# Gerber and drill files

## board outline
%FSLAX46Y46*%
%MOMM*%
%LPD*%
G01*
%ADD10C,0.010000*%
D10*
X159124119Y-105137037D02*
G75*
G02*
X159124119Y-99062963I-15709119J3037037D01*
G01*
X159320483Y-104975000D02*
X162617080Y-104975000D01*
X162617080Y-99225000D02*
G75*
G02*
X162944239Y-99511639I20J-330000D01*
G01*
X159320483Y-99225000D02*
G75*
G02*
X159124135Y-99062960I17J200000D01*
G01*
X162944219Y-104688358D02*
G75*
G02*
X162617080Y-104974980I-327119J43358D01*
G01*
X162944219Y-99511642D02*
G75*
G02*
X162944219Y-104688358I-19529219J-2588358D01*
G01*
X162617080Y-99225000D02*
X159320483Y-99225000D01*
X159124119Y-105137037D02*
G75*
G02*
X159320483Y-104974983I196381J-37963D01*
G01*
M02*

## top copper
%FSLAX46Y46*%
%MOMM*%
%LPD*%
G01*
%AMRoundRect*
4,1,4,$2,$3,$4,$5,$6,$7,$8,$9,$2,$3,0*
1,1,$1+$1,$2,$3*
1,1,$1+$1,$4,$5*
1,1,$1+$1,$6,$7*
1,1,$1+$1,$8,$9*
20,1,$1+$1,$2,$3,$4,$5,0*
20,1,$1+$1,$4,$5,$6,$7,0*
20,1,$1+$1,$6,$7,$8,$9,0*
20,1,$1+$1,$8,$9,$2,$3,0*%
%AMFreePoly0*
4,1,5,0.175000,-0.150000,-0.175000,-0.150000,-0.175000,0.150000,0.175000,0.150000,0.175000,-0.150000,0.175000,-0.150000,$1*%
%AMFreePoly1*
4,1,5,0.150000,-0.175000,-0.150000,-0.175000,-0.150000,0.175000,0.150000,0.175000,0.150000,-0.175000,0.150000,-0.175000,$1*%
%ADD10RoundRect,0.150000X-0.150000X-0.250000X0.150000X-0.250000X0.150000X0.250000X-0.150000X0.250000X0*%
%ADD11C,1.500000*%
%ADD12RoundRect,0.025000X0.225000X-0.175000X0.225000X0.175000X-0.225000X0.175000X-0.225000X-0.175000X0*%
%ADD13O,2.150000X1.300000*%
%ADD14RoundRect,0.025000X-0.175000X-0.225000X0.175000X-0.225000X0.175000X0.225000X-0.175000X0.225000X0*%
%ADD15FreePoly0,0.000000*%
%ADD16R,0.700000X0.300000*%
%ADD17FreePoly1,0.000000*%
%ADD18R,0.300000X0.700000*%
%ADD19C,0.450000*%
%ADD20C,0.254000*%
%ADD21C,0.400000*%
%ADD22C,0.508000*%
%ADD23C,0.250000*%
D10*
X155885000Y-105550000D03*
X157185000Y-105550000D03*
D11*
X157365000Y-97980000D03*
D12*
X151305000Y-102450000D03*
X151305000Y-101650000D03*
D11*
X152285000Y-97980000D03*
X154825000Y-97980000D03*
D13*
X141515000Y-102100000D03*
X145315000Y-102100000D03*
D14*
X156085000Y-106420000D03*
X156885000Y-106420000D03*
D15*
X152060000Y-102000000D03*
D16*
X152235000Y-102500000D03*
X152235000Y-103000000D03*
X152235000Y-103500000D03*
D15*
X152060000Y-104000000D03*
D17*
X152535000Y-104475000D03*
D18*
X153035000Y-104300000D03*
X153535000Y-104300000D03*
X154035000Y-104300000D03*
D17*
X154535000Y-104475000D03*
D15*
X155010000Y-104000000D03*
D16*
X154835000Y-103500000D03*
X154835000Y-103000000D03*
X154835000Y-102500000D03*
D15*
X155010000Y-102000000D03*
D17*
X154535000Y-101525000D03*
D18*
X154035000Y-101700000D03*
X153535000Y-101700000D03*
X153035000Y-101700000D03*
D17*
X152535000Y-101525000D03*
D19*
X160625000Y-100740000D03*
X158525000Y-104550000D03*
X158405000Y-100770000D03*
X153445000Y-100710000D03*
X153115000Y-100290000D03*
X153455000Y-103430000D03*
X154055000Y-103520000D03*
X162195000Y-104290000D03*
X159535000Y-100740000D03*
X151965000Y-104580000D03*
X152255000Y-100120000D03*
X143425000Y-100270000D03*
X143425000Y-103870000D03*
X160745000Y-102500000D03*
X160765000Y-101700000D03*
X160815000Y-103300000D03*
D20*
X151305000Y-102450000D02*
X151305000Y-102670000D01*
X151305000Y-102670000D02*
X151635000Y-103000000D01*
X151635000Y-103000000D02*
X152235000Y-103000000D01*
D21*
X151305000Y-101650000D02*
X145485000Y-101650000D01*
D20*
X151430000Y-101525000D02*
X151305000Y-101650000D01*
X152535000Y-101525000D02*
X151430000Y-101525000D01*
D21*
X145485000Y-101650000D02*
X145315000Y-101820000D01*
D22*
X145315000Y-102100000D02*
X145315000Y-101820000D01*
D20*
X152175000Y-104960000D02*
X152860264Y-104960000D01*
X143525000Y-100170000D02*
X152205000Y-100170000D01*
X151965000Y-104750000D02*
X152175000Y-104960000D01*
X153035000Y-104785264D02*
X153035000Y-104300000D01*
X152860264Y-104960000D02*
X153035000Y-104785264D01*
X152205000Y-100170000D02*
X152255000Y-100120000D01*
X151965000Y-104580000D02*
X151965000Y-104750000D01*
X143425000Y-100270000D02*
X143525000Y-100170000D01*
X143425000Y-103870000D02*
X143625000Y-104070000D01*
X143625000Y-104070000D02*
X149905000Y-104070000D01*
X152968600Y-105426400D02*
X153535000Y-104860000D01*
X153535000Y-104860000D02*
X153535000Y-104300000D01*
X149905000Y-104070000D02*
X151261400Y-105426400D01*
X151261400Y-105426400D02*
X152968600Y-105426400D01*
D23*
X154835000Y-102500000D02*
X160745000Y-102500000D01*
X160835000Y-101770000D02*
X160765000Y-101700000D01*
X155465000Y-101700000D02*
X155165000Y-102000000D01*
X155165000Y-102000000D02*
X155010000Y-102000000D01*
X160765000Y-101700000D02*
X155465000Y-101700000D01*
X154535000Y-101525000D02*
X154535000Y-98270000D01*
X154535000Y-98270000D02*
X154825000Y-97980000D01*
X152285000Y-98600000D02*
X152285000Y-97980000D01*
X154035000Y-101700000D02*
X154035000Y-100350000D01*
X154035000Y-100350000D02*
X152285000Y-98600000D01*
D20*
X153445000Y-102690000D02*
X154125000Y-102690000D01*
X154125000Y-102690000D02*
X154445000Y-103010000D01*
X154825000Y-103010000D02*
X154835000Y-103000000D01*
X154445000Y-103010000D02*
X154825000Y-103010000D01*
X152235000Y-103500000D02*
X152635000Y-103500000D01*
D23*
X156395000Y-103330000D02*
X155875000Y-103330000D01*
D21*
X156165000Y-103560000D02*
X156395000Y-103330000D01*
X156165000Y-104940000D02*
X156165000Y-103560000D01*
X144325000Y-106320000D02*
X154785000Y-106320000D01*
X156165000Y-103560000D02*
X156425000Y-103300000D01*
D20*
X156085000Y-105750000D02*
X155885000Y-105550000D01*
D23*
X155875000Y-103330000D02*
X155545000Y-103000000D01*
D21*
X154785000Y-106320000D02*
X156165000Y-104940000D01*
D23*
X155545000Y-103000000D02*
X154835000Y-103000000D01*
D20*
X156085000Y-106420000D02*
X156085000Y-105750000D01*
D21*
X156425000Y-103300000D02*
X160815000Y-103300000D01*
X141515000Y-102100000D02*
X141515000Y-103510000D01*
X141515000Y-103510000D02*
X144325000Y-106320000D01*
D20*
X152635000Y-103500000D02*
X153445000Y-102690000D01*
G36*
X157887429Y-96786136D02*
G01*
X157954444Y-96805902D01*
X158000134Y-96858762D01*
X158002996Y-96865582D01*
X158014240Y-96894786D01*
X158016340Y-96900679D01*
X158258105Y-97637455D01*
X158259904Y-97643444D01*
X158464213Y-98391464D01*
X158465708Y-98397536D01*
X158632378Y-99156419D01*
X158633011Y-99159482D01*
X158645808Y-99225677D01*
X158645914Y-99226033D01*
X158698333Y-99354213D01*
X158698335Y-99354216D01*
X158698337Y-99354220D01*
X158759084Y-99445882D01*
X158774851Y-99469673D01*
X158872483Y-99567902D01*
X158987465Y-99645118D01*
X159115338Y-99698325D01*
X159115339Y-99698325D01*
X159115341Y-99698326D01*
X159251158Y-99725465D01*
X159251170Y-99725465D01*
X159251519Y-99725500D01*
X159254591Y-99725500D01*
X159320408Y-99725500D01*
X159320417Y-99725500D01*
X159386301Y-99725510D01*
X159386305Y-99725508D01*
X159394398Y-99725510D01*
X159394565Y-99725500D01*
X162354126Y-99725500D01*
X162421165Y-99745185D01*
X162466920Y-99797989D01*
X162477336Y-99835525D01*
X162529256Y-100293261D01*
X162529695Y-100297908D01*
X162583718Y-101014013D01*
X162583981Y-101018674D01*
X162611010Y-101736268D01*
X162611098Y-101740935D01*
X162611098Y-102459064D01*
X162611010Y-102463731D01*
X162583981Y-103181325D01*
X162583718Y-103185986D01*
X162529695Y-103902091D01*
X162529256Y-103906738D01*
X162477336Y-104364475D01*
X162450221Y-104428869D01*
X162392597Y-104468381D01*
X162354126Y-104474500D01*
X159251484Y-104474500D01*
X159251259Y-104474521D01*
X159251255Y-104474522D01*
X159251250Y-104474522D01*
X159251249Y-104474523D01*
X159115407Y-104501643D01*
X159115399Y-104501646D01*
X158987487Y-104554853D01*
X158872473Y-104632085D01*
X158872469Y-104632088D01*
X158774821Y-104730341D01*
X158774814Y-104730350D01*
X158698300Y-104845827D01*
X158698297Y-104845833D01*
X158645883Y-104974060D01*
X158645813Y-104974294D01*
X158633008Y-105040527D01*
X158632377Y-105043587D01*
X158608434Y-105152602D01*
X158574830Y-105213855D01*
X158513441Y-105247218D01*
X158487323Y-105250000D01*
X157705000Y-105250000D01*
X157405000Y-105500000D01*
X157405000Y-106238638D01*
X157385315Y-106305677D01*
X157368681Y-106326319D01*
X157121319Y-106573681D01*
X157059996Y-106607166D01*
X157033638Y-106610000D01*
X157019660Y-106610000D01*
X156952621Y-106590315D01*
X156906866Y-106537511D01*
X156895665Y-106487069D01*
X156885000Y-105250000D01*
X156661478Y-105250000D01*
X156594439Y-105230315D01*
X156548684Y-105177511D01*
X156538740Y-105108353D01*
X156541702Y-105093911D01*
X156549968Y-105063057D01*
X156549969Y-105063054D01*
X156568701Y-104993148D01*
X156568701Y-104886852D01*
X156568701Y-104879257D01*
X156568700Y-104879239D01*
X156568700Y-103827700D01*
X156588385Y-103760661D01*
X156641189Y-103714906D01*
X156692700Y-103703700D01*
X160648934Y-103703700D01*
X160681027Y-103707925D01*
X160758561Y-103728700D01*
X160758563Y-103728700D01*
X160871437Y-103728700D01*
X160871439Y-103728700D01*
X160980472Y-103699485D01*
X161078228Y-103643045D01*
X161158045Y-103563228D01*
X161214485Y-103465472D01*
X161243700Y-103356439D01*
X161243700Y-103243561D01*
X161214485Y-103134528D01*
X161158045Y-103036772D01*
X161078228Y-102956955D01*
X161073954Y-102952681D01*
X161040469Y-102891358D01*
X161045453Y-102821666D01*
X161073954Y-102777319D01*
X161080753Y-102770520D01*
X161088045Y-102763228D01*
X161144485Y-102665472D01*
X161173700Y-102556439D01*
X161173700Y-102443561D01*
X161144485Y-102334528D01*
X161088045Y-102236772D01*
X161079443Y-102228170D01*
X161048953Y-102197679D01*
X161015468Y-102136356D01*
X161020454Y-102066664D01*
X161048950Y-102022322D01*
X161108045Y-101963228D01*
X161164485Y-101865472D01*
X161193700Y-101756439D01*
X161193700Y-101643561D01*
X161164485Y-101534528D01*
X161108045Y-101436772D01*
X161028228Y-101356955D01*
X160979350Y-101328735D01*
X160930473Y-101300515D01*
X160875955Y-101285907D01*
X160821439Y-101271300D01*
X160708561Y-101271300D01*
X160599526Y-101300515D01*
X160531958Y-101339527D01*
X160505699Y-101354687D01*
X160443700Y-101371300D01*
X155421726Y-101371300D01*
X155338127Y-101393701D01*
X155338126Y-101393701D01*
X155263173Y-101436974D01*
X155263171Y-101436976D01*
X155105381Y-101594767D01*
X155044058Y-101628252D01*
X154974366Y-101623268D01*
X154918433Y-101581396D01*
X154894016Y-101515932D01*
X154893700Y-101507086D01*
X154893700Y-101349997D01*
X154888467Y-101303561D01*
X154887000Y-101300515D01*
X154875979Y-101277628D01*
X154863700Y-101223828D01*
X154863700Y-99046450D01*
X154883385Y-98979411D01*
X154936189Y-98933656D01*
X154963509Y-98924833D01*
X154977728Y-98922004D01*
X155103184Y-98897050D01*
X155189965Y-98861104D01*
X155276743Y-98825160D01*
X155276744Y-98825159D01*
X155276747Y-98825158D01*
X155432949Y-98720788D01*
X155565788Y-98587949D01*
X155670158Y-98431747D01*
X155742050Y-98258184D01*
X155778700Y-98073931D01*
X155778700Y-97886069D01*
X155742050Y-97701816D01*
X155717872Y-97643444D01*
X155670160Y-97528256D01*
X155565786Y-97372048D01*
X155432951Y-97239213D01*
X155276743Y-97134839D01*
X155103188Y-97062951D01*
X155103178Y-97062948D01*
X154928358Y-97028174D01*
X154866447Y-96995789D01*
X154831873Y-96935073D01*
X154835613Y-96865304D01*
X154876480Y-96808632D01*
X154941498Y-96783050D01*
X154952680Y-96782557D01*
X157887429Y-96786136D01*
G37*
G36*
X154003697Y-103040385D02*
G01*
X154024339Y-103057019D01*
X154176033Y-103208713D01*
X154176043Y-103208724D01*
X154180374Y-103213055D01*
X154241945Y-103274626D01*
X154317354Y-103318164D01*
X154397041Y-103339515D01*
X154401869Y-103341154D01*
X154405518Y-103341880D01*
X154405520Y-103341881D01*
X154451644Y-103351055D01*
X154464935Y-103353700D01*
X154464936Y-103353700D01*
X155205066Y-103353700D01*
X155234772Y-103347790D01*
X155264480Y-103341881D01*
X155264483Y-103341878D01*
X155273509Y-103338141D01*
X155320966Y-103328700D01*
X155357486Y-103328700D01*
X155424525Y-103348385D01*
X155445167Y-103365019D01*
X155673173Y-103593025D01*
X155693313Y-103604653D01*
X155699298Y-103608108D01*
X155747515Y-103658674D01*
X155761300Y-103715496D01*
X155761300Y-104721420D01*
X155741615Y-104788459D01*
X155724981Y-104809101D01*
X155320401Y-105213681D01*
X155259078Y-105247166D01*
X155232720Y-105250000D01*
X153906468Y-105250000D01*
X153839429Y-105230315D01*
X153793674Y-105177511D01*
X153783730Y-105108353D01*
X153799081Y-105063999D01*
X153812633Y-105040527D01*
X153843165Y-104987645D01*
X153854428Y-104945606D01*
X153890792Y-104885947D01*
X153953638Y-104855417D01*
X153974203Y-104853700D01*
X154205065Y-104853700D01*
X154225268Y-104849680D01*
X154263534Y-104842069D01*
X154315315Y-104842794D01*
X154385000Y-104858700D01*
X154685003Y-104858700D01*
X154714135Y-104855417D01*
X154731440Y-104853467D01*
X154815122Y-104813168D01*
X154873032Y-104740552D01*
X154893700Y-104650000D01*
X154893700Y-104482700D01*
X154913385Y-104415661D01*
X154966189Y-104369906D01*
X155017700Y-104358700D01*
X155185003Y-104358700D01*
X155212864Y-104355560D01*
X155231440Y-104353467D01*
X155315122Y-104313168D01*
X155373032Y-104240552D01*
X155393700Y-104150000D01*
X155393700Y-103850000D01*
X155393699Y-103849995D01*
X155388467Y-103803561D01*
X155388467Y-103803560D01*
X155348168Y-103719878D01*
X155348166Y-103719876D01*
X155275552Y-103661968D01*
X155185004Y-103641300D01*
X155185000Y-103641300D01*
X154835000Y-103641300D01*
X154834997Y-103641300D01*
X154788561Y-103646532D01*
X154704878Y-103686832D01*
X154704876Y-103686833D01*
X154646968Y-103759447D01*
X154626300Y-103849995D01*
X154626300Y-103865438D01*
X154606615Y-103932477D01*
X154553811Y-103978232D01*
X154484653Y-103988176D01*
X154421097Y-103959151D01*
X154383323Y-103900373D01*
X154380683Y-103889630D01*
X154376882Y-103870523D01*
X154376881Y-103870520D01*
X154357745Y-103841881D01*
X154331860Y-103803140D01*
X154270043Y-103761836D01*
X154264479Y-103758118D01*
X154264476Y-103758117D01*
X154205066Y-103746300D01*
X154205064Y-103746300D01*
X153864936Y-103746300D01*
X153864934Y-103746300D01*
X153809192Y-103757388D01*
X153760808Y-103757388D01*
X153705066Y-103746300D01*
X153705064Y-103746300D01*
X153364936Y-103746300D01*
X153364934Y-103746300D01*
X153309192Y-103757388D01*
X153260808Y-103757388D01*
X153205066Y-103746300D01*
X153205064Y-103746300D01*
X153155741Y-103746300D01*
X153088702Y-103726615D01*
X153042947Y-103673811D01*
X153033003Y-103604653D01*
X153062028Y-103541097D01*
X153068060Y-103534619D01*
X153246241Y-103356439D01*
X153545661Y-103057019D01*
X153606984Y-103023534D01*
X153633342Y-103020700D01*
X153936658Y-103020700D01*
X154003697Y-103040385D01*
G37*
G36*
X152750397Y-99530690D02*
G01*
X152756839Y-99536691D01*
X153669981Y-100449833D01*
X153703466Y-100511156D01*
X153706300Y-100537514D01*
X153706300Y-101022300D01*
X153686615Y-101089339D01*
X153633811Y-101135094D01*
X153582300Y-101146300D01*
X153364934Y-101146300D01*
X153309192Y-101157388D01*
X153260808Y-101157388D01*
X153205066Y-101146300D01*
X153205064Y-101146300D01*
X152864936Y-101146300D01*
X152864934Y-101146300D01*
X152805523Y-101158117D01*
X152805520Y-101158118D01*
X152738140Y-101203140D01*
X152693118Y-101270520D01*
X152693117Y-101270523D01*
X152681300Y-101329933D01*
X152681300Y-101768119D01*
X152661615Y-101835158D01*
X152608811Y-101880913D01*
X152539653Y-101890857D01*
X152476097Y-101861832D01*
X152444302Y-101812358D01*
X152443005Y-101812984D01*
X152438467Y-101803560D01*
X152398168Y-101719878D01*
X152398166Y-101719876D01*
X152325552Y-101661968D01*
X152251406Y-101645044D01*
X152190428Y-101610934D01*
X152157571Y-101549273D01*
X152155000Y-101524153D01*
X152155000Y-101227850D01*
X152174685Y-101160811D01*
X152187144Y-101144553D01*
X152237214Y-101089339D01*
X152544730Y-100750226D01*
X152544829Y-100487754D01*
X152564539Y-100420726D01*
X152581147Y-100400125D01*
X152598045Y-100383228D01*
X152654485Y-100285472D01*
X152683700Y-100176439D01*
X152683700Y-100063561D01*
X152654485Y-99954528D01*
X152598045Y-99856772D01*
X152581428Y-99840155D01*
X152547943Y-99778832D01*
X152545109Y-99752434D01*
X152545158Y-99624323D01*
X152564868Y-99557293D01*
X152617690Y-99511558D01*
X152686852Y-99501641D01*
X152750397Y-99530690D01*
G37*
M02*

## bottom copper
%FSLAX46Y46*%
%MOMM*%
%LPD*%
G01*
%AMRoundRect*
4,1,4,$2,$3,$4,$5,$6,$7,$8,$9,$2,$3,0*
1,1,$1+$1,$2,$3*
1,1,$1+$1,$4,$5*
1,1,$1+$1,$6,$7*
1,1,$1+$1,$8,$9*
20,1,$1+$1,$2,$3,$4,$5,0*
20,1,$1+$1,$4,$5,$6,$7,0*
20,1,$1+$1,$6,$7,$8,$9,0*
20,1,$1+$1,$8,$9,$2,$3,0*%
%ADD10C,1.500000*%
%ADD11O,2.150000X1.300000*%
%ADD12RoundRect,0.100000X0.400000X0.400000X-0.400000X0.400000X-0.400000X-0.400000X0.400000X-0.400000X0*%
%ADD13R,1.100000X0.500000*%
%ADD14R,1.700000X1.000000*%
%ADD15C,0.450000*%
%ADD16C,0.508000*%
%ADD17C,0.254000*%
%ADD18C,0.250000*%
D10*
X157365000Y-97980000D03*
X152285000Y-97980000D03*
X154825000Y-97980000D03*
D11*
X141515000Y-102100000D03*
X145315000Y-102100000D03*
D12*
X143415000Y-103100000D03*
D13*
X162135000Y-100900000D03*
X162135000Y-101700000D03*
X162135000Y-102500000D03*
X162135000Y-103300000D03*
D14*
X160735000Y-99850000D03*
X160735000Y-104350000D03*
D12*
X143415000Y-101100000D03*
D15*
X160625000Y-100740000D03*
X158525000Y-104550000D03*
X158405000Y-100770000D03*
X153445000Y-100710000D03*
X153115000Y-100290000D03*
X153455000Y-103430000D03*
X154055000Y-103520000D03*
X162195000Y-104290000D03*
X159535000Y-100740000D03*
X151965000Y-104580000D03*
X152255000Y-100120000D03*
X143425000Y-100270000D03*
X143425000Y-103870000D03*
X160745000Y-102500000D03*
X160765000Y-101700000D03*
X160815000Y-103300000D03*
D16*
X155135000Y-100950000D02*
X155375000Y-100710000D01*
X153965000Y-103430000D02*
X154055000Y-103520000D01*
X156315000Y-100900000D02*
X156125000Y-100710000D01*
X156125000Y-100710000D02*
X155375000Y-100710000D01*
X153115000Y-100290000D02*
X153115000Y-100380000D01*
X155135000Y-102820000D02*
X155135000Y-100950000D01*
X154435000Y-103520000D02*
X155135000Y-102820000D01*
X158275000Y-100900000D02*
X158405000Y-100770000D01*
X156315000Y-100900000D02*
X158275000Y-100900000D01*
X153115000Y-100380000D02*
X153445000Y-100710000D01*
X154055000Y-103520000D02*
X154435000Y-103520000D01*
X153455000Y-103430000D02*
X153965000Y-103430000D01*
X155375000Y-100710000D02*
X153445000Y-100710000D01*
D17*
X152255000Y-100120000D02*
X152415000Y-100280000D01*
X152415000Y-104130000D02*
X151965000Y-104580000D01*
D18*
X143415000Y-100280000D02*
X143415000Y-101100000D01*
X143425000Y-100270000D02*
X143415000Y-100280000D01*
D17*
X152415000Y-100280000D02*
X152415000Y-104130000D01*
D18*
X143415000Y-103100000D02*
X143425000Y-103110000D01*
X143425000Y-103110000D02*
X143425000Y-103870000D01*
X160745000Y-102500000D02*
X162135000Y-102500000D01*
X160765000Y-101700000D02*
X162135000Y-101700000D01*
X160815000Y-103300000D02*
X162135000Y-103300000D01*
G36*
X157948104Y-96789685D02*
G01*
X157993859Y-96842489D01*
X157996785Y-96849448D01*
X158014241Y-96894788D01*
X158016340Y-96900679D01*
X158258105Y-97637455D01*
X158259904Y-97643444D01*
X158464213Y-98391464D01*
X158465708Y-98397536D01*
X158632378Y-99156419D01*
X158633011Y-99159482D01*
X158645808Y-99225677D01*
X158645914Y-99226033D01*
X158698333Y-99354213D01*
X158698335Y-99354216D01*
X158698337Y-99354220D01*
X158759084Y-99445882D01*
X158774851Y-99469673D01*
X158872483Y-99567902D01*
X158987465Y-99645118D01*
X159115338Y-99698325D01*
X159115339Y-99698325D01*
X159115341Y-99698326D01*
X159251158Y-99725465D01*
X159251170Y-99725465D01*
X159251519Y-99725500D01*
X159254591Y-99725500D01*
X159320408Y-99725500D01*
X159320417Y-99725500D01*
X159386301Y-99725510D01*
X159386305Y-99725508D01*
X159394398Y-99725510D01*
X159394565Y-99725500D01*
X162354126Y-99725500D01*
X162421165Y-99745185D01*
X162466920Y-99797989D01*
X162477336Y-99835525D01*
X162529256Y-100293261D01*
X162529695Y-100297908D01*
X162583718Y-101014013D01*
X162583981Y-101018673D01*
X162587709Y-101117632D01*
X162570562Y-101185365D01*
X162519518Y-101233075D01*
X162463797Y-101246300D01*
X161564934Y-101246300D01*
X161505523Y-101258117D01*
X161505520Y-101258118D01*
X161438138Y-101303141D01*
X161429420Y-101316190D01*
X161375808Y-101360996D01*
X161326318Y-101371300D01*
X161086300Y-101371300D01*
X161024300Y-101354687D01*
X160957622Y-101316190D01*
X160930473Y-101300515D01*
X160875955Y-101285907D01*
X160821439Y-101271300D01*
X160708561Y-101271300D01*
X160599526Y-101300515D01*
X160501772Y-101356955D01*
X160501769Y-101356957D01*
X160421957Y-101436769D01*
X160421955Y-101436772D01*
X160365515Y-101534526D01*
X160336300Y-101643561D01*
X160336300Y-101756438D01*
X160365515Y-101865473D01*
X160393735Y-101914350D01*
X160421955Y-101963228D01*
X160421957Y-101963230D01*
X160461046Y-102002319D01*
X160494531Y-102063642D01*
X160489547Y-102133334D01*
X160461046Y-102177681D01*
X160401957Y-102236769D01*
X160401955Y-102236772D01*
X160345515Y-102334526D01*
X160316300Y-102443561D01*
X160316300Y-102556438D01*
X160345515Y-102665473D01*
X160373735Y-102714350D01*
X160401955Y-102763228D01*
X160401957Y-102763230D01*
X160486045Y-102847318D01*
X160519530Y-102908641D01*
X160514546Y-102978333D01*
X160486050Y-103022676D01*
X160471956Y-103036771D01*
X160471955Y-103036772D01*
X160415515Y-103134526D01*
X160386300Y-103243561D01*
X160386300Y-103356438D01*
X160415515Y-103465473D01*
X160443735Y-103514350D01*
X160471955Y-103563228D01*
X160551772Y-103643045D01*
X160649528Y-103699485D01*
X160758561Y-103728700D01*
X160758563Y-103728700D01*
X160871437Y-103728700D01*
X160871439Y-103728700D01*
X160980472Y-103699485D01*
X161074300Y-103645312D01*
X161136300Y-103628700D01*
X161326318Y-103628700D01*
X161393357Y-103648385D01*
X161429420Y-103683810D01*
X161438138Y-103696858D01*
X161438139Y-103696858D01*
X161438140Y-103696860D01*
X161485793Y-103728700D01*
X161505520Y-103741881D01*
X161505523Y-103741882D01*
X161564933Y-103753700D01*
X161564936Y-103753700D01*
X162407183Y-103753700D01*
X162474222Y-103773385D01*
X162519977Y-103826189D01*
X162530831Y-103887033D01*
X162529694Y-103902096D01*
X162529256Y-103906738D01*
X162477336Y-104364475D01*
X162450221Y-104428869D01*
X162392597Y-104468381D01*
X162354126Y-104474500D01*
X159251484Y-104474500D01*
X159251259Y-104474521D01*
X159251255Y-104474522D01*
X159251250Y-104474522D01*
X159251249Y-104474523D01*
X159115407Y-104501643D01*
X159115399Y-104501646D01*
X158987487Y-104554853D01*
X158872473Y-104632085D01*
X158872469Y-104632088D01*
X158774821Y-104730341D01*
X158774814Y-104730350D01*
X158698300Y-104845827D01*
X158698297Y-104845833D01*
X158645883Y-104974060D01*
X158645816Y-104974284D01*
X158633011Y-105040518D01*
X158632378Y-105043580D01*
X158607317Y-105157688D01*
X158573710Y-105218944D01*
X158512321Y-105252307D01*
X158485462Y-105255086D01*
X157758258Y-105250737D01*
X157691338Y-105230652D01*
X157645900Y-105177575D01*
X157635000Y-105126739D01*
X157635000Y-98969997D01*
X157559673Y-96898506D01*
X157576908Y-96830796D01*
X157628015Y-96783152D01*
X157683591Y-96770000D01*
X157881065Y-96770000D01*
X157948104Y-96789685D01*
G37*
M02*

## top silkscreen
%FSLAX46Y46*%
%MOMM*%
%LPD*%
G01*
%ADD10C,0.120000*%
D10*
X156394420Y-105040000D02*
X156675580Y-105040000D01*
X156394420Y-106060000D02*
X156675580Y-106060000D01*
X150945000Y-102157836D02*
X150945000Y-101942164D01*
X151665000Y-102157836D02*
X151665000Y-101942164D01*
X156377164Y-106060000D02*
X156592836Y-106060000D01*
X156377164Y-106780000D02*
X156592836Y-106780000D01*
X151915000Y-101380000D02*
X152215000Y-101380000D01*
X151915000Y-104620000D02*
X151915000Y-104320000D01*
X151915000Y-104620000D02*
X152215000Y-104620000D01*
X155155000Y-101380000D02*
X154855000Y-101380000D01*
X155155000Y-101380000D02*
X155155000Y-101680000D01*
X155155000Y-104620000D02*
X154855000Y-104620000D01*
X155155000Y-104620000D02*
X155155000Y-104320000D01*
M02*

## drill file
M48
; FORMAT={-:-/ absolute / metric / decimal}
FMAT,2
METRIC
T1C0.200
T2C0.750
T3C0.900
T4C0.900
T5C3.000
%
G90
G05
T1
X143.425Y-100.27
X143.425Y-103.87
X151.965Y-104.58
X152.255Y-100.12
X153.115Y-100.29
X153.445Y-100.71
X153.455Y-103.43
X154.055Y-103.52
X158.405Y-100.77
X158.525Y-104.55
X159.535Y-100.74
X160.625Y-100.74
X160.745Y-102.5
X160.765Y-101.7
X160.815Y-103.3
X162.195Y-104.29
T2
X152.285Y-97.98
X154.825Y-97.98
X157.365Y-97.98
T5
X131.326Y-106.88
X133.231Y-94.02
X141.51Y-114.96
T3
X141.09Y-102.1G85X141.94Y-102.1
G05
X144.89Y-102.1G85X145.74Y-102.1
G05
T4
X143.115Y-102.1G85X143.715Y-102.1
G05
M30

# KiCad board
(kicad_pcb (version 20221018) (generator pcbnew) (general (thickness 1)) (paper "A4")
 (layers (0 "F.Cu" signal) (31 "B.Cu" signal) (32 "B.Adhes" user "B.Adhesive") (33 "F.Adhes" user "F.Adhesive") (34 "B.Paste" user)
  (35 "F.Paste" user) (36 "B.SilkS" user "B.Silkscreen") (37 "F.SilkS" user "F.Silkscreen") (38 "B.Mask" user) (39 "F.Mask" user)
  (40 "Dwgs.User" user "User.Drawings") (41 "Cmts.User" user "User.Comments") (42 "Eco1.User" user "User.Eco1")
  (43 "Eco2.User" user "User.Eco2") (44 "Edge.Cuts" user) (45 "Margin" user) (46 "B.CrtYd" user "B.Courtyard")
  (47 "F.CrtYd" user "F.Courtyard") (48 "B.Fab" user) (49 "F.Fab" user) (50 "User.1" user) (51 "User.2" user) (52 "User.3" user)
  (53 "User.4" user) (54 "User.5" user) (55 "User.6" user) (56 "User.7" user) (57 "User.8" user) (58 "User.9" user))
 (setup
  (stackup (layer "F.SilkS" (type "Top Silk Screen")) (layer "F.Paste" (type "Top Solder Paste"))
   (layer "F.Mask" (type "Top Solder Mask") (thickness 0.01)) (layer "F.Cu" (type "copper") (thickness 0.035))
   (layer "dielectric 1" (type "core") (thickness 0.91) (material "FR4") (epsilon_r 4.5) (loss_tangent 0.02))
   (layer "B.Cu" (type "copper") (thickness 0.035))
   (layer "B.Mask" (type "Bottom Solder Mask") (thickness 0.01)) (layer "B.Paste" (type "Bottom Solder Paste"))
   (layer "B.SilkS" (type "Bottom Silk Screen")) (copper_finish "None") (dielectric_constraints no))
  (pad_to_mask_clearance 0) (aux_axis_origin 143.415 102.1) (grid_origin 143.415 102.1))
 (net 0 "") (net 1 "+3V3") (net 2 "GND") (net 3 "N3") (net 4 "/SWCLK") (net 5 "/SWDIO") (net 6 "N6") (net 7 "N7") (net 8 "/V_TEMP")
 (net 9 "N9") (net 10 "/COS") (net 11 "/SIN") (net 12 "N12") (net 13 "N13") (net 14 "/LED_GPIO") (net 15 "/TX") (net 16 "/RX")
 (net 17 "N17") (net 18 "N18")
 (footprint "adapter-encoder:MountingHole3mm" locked (layer "F.Cu") (at 141.509772 114.959631)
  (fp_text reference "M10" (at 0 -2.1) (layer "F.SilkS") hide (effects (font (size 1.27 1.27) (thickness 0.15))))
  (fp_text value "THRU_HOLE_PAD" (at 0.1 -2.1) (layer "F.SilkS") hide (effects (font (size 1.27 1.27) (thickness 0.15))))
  (pad "" np_thru_hole oval locked (at 0 0) (size 3 3) (drill 3) (layers "*.Mask") (thermal_bridge_angle 45)))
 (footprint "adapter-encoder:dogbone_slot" (layer "F.Cu") (at 143.415 102.1)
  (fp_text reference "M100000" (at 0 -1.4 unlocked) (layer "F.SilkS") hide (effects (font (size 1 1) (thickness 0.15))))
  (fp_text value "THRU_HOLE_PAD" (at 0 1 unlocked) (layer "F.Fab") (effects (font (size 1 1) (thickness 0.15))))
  (pad "" np_thru_hole oval (at 0 0) (size 1.5 0.9) (drill oval 1.5 0.9) (layers "*.Mask") (thermal_bridge_angle 45)))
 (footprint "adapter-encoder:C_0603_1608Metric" (layer "F.Cu") (at 156.535 105.55)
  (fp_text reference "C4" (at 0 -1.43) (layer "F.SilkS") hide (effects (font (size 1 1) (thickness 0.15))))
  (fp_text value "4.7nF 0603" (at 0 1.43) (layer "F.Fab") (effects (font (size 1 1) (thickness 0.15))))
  (fp_line (start -0.14058 -0.51) (end 0.14058 -0.51) (stroke (width 0.12) (type solid)) (layer "F.SilkS"))
  (fp_line (start -0.14058 0.51) (end 0.14058 0.51) (stroke (width 0.12) (type solid)) (layer "F.SilkS"))
  (pad "1" smd roundrect (at -0.65 0) (size 0.6 0.8) (layers "F.Cu" "F.Paste" "F.Mask") (roundrect_rratio 0.25) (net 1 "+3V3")
   (solder_mask_margin 0.0508))
  (pad "2" smd roundrect (at 0.65 0) (size 0.6 0.8) (layers "F.Cu" "F.Paste" "F.Mask") (roundrect_rratio 0.25) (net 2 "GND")
   (solder_mask_margin 0.0508)))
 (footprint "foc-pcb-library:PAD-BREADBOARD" (layer "F.Cu") (at 157.365 97.98)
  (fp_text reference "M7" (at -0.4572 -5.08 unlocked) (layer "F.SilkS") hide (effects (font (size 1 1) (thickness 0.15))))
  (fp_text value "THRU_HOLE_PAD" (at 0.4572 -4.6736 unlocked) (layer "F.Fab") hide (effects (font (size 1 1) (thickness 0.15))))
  (pad "1" thru_hole circle (at 0 0) (size 1.5 1.5) (drill 0.75) (layers "*.Cu" "*.Mask") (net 2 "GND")))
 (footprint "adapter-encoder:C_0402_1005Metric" (layer "F.Cu") (at 151.305 102.05 90)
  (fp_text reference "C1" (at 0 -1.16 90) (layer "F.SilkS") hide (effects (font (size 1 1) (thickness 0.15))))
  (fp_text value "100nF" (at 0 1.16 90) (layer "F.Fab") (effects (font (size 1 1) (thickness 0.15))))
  (fp_line (start -0.107836 -0.36) (end 0.107836 -0.36) (stroke (width 0.12) (type solid)) (layer "F.SilkS"))
  (fp_line (start -0.107836 0.36) (end 0.107836 0.36) (stroke (width 0.12) (type solid)) (layer "F.SilkS"))
  (pad "1" smd roundrect (at -0.4 0 90) (size 0.4 0.5) (layers "F.Cu" "F.Paste" "F.Mask") (roundrect_rratio 0.0625) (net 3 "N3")
   (solder_mask_margin 0.0508))
  (pad "2" smd roundrect (at 0.4 0 90) (size 0.4 0.5) (layers "F.Cu" "F.Paste" "F.Mask") (roundrect_rratio 0.0625) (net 2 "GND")
   (solder_mask_margin 0.0508)))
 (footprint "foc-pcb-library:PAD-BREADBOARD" (layer "F.Cu") (at 152.285 97.98)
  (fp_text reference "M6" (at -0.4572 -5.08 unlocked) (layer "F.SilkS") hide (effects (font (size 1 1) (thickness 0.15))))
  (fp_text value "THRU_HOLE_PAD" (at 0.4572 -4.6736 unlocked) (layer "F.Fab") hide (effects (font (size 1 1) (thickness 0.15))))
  (pad "1" thru_hole circle (at 0 0) (size 1.5 1.5) (drill 0.75) (layers "*.Cu" "*.Mask") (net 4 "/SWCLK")))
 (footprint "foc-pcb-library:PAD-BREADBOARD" (layer "F.Cu") (at 154.825 97.98)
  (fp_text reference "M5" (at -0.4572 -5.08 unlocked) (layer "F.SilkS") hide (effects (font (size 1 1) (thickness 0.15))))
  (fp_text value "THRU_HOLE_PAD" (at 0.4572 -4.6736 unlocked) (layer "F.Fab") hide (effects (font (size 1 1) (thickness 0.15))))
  (pad "1" thru_hole circle (at 0 0) (size 1.5 1.5) (drill 0.75) (layers "*.Cu" "*.Mask") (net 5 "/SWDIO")))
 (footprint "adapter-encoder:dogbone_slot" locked (layer "F.Cu") (at 141.515 102.1)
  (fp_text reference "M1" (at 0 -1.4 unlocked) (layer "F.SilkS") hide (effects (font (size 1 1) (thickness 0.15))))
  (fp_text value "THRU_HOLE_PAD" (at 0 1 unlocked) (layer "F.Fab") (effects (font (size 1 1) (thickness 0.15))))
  (pad "1" thru_hole oval locked (at 0 0) (size 2.15 1.3) (drill oval 1.75 0.9) (layers "*.Cu" "*.Mask") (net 1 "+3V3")
   (thermal_bridge_angle 45)))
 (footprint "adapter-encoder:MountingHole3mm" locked (layer "F.Cu") (at 133.230847 94.02021)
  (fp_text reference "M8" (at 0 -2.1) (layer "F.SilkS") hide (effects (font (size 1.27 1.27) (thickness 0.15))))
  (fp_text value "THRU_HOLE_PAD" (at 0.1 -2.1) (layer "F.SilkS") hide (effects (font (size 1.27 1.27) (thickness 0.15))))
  (pad "" np_thru_hole oval locked (at 0 0) (size 3 3) (drill 3) (layers "*.Mask") (thermal_bridge_angle 45)))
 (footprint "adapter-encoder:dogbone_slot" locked (layer "F.Cu") (at 145.315 102.1)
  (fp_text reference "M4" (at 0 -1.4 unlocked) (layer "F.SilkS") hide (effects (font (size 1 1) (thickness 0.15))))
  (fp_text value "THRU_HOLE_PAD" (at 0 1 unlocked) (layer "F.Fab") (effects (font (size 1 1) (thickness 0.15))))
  (pad "1" thru_hole oval locked (at 0 0) (size 2.15 1.3) (drill oval 1.75 0.9) (layers "*.Cu" "*.Mask") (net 2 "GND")
   (thermal_bridge_angle 45)))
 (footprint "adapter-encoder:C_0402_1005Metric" (layer "F.Cu") (at 156.485 106.42)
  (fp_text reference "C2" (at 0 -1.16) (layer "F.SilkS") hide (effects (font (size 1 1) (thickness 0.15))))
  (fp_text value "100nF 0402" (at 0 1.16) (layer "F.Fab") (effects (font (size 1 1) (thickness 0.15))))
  (fp_line (start -0.107836 -0.36) (end 0.107836 -0.36) (stroke (width 0.12) (type solid)) (layer "F.SilkS"))
  (fp_line (start -0.107836 0.36) (end 0.107836 0.36) (stroke (width 0.12) (type solid)) (layer "F.SilkS"))
  (pad "1" smd roundrect (at -0.4 0) (size 0.4 0.5) (layers "F.Cu" "F.Paste" "F.Mask") (roundrect_rratio 0.0625) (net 1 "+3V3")
   (solder_mask_margin 0.0508))
  (pad "2" smd roundrect (at 0.4 0) (size 0.4 0.5) (layers "F.Cu" "F.Paste" "F.Mask") (roundrect_rratio 0.0625) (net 2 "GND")
   (solder_mask_margin 0.0508)))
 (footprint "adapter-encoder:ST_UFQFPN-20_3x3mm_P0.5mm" (layer "F.Cu") (at 153.535 103)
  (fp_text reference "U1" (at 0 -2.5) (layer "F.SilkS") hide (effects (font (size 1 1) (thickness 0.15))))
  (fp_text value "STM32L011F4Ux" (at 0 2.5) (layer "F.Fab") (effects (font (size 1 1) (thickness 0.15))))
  (fp_line (start -1.62 -1.62) (end -1.32 -1.62) (stroke (width 0.12) (type solid)) (layer "F.SilkS"))
  (fp_line (start -1.62 1.62) (end -1.62 1.32) (stroke (width 0.12) (type solid)) (layer "F.SilkS"))
  (fp_line (start -1.62 1.62) (end -1.32 1.62) (stroke (width 0.12) (type solid)) (layer "F.SilkS"))
  (fp_line (start 1.62 -1.62) (end 1.32 -1.62) (stroke (width 0.12) (type solid)) (layer "F.SilkS"))
  (fp_line (start 1.62 -1.62) (end 1.62 -1.32) (stroke (width 0.12) (type solid)) (layer "F.SilkS"))
  (fp_line (start 1.62 1.62) (end 1.32 1.62) (stroke (width 0.12) (type solid)) (layer "F.SilkS"))
  (fp_line (start 1.62 1.62) (end 1.62 1.32) (stroke (width 0.12) (type solid)) (layer "F.SilkS"))
  (pad "1" smd custom (at -1.475 -1) (size 0.35 0.3) (layers "F.Cu" "F.Paste" "F.Mask") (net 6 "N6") (zone_connect 2)
   (options (clearance outline) (anchor rect)) (primitives))
  (pad "2" smd rect (at -1.3 -0.5) (size 0.7 0.3) (layers "F.Cu" "F.Paste" "F.Mask") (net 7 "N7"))
  (pad "3" smd rect (at -1.3 0) (size 0.7 0.3) (layers "F.Cu" "F.Paste" "F.Mask") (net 3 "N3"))
  (pad "4" smd rect (at -1.3 0.5) (size 0.7 0.3) (layers "F.Cu" "F.Paste" "F.Mask") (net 1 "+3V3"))
  (pad "5" smd custom (at -1.475 1) (size 0.35 0.3) (layers "F.Cu" "F.Paste" "F.Mask") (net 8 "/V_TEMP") (zone_connect 2)
   (options (clearance outline) (anchor rect)) (primitives))
  (pad "6" smd custom (at -1 1.475) (size 0.3 0.35) (layers "F.Cu" "F.Paste" "F.Mask") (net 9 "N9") (zone_connect 2)
   (options (clearance outline) (anchor rect)) (primitives))
  (pad "7" smd rect (at -0.5 1.3) (size 0.3 0.7) (layers "F.Cu" "F.Paste" "F.Mask") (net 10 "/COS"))
  (pad "8" smd rect (at 0 1.3) (size 0.3 0.7) (layers "F.Cu" "F.Paste" "F.Mask") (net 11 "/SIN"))
  (pad "9" smd rect (at 0.5 1.3) (size 0.3 0.7) (layers "F.Cu" "F.Paste" "F.Mask") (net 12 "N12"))
  (pad "10" smd custom (at 1 1.475) (size 0.3 0.35) (layers "F.Cu" "F.Paste" "F.Mask") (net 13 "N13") (zone_connect 2)
   (options (clearance outline) (anchor rect)) (primitives))
  (pad "11" smd custom (at 1.475 1) (size 0.35 0.3) (layers "F.Cu" "F.Paste" "F.Mask") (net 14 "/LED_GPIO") (zone_connect 2)
   (options (clearance outline) (anchor rect)) (primitives))
  (pad "12" smd rect (at 1.3 0.5) (size 0.7 0.3) (layers "F.Cu" "F.Paste" "F.Mask") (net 2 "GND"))
  (pad "13" smd rect (at 1.3 0) (size 0.7 0.3) (layers "F.Cu" "F.Paste" "F.Mask") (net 1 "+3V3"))
  (pad "14" smd rect (at 1.3 -0.5) (size 0.7 0.3) (layers "F.Cu" "F.Paste" "F.Mask") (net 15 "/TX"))
  (pad "15" smd custom (at 1.475 -1) (size 0.35 0.3) (layers "F.Cu" "F.Paste" "F.Mask") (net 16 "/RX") (zone_connect 2)
   (options (clearance outline) (anchor rect)) (primitives))
  (pad "16" smd custom (at 1 -1.475) (size 0.3 0.35) (layers "F.Cu" "F.Paste" "F.Mask") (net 5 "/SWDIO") (zone_connect 2)
   (options (clearance outline) (anchor rect)) (primitives))
  (pad "17" smd rect (at 0.5 -1.3) (size 0.3 0.7) (layers "F.Cu" "F.Paste" "F.Mask") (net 4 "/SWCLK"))
  (pad "18" smd rect (at 0 -1.3) (size 0.3 0.7) (layers "F.Cu" "F.Paste" "F.Mask") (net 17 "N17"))
  (pad "19" smd rect (at -0.5 -1.3) (size 0.3 0.7) (layers "F.Cu" "F.Paste" "F.Mask") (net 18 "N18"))
  (pad "20" smd custom (at -1 -1.475) (size 0.3 0.35) (layers "F.Cu" "F.Paste" "F.Mask") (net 2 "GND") (zone_connect 2)
   (options (clearance outline) (anchor rect)) (primitives)))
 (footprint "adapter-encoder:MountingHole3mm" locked (layer "F.Cu") (at 131.325619 106.87984)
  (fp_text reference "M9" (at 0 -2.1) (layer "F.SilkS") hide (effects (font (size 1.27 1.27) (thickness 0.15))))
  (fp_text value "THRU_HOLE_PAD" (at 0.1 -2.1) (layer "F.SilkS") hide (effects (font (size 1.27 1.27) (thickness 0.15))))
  (pad "" np_thru_hole oval locked (at 0 0) (size 3 3) (drill 3) (layers "*.Mask") (thermal_bridge_angle 45)))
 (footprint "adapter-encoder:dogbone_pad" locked (layer "B.Cu") (at 143.415 103.1 180)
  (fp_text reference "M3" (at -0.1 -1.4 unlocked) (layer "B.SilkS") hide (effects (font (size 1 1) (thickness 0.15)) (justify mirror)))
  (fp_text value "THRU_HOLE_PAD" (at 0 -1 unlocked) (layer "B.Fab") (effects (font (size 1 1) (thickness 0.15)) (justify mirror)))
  (pad "1" smd roundrect locked (at 0 0 180) (size 1 1) (layers "B.Cu" "B.Paste" "B.Mask") (roundrect_rratio 0.1) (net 11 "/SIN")
   (thermal_bridge_angle 45)))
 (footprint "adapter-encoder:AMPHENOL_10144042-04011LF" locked (layer "B.Cu") (at 162.135 102.1 90)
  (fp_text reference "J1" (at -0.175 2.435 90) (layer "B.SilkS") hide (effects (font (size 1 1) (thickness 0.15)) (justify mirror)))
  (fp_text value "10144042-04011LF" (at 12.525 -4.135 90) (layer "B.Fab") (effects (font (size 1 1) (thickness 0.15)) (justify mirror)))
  (pad "1" smd rect locked (at 1.2 0 90) (size 0.5 1.1) (layers "B.Cu" "B.Paste" "B.Mask") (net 2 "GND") (solder_mask_margin 0.102))
  (pad "2" smd rect locked (at 0.4 0 90) (size 0.5 1.1) (layers "B.Cu" "B.Paste" "B.Mask") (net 16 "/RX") (solder_mask_margin 0.102))
  (pad "3" smd rect locked (at -0.4 0 90) (size 0.5 1.1) (layers "B.Cu" "B.Paste" "B.Mask") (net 15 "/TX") (solder_mask_margin 0.102))
  (pad "4" smd rect locked (at -1.2 0 90) (size 0.5 1.1) (layers "B.Cu" "B.Paste" "B.Mask") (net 1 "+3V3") (solder_mask_margin 0.102))
  (pad "S1" smd rect locked (at 2.25 -1.4 90) (size 1 1.7) (layers "B.Cu" "B.Paste" "B.Mask") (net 2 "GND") (solder_mask_margin 0.102))
  (pad "S2" smd rect locked (at -2.25 -1.4 90) (size 1 1.7) (layers "B.Cu" "B.Paste" "B.Mask") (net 2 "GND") (solder_mask_margin 0.102)))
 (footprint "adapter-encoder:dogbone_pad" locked (layer "B.Cu") (at 143.415 101.1 180)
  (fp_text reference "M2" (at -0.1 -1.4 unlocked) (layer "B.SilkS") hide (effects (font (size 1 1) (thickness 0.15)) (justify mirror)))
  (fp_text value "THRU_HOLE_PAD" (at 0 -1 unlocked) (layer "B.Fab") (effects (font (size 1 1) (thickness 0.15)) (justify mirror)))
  (pad "1" smd roundrect locked (at 0 0 180) (size 1 1) (layers "B.Cu" "B.Paste" "B.Mask") (roundrect_rratio 0.1) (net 10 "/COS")
   (thermal_bridge_angle 45)))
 (gr_arc locked (start 159.124119 105.137037) (mid 127.415 102.1) (end 159.124119 99.062963) (stroke (width 0.01) (type solid))
  (layer "Edge.Cuts"))
 (gr_line locked (start 159.320483 104.975) (end 162.61708 104.975) (stroke (width 0.01) (type solid)) (layer "Edge.Cuts"))
 (gr_arc locked (start 162.61708 99.225) (mid 162.834568 99.306791) (end 162.944219 99.511642) (stroke (width 0.01) (type solid))
  (layer "Edge.Cuts"))
 (gr_arc locked (start 159.320483 99.225) (mid 159.193198 99.179254) (end 159.124119 99.062963) (stroke (width 0.01) (type solid))
  (layer "Edge.Cuts"))
 (gr_arc locked (start 162.944219 104.688358) (mid 162.834555 104.893194) (end 162.61708 104.975) (stroke (width 0.01) (type solid))
  (layer "Edge.Cuts"))
 (gr_arc locked (start 162.944219 99.511642) (mid 163.115 102.1) (end 162.944219 104.688358) (stroke (width 0.01) (type solid))
  (layer "Edge.Cuts"))
 (gr_line locked (start 162.61708 99.225) (end 159.320483 99.225) (stroke (width 0.01) (type solid)) (layer "Edge.Cuts"))
 (gr_arc locked (start 159.124119 105.137037) (mid 159.193188 105.020733) (end 159.320483 104.975) (stroke (width 0.01) (type solid))
  (layer "Edge.Cuts"))
 (segment (start 151.305 102.45) (end 151.305 102.67) (width 0.254) (layer "F.Cu") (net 3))
 (segment (start 151.305 102.67) (end 151.635 103) (width 0.254) (layer "F.Cu") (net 3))
 (segment (start 151.635 103) (end 152.235 103) (width 0.254) (layer "F.Cu") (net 3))
 (segment (start 151.305 101.65) (end 145.485 101.65) (width 0.4) (layer "F.Cu") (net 2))
 (segment (start 151.43 101.525) (end 151.305 101.65) (width 0.254) (layer "F.Cu") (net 2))
 (segment (start 152.535 101.525) (end 151.43 101.525) (width 0.254) (layer "F.Cu") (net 2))
 (segment (start 145.485 101.65) (end 145.315 101.82) (width 0.4) (layer "F.Cu") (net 2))
 (segment (start 145.315 102.1) (end 145.315 101.82) (width 0.508) (layer "F.Cu") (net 2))
 (via (at 160.625 100.74) (size 0.45) (drill 0.2) (layers "F.Cu" "B.Cu") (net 2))
 (via (at 158.525 104.55) (size 0.45) (drill 0.2) (layers "F.Cu" "B.Cu") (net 2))
 (via (at 158.405 100.77) (size 0.45) (drill 0.2) (layers "F.Cu" "B.Cu") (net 2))
 (via (at 153.445 100.71) (size 0.45) (drill 0.2) (layers "F.Cu" "B.Cu") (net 2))
 (via (at 153.115 100.29) (size 0.45) (drill 0.2) (layers "F.Cu" "B.Cu") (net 2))
 (via (at 153.455 103.43) (size 0.45) (drill 0.2) (layers "F.Cu" "B.Cu") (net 2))
 (via (at 154.055 103.52) (size 0.45) (drill 0.2) (layers "F.Cu" "B.Cu") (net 2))
 (via (at 162.195 104.29) (size 0.45) (drill 0.2) (layers "F.Cu" "B.Cu") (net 2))
 (via (at 159.535 100.74) (size 0.45) (drill 0.2) (layers "F.Cu" "B.Cu") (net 2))
 (segment (start 155.135 100.95) (end 155.375 100.71) (width 0.508) (layer "B.Cu") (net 2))
 (segment (start 153.965 103.43) (end 154.055 103.52) (width 0.508) (layer "B.Cu") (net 2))
 (segment (start 156.315 100.9) (end 156.125 100.71) (width 0.508) (layer "B.Cu") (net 2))
 (segment (start 156.125 100.71) (end 155.375 100.71) (width 0.508) (layer "B.Cu") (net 2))
 (segment (start 153.115 100.29) (end 153.115 100.38) (width 0.508) (layer "B.Cu") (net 2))
 (segment (start 155.135 102.82) (end 155.135 100.95) (width 0.508) (layer "B.Cu") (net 2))
 (segment (start 154.435 103.52) (end 155.135 102.82) (width 0.508) (layer "B.Cu") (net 2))
 (segment (start 158.275 100.9) (end 158.405 100.77) (width 0.508) (layer "B.Cu") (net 2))
 (segment (start 156.315 100.9) (end 158.275 100.9) (width 0.508) (layer "B.Cu") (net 2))
 (segment (start 153.115 100.38) (end 153.445 100.71) (width 0.508) (layer "B.Cu") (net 2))
 (segment (start 154.055 103.52) (end 154.435 103.52) (width 0.508) (layer "B.Cu") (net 2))
 (segment (start 153.455 103.43) (end 153.965 103.43) (width 0.508) (layer "B.Cu") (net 2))
 (segment (start 155.375 100.71) (end 153.445 100.71) (width 0.508) (layer "B.Cu") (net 2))
 (segment (start 152.175 104.96) (end 152.860264 104.96) (width 0.254) (layer "F.Cu") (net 10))
 (segment (start 143.525 100.17) (end 152.205 100.17) (width 0.254) (layer "F.Cu") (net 10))
 (segment (start 151.965 104.75) (end 152.175 104.96) (width 0.254) (layer "F.Cu") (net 10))
 (segment (start 153.035 104.785264) (end 153.035 104.3) (width 0.254) (layer "F.Cu") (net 10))
 (segment (start 152.860264 104.96) (end 153.035 104.785264) (width 0.254) (layer "F.Cu") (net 10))
 (segment (start 152.205 100.17) (end 152.255 100.12) (width 0.254) (layer "F.Cu") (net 10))
 (segment (start 151.965 104.58) (end 151.965 104.75) (width 0.254) (layer "F.Cu") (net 10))
 (segment (start 143.425 100.27) (end 143.525 100.17) (width 0.254) (layer "F.Cu") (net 10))
 (via (at 151.965 104.58) (size 0.45) (drill 0.2) (layers "F.Cu" "B.Cu") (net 10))
 (via (at 152.255 100.12) (size 0.45) (drill 0.2) (layers "F.Cu" "B.Cu") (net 10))
 (via (at 143.425 100.27) (size 0.45) (drill 0.2) (layers "F.Cu" "B.Cu") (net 10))
 (segment (start 152.255 100.12) (end 152.415 100.28) (width 0.254) (layer "B.Cu") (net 10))
 (segment (start 152.415 104.13) (end 151.965 104.58) (width 0.254) (layer "B.Cu") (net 10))
 (segment (start 143.415 100.28) (end 143.415 101.1) (width 0.25) (layer "B.Cu") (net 10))
 (segment (start 143.425 100.27) (end 143.415 100.28) (width 0.25) (layer "B.Cu") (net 10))
 (segment (start 152.415 100.28) (end 152.415 104.13) (width 0.254) (layer "B.Cu") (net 10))
 (segment (start 143.425 103.87) (end 143.625 104.07) (width 0.254) (layer "F.Cu") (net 11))
 (segment (start 143.625 104.07) (end 149.905 104.07) (width 0.254) (layer "F.Cu") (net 11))
 (segment (start 152.9686 105.4264) (end 153.535 104.86) (width 0.254) (layer "F.Cu") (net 11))
 (segment (start 153.535 104.86) (end 153.535 104.3) (width 0.254) (layer "F.Cu") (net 11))
 (segment (start 149.905 104.07) (end 151.2614 105.4264) (width 0.254) (layer "F.Cu") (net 11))
 (segment (start 151.2614 105.4264) (end 152.9686 105.4264) (width 0.254) (layer "F.Cu") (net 11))
 (via (at 143.425 103.87) (size 0.45) (drill 0.2) (layers "F.Cu" "B.Cu") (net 11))
 (segment (start 143.415 103.1) (end 143.425 103.11) (width 0.25) (layer "B.Cu") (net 11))
 (segment (start 143.425 103.11) (end 143.425 103.87) (width 0.25) (layer "B.Cu") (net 11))
 (segment (start 154.835 102.5) (end 160.745 102.5) (width 0.25) (layer "F.Cu") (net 15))
 (via (at 160.745 102.5) (size 0.45) (drill 0.2) (layers "F.Cu" "B.Cu") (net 15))
 (segment (start 160.745 102.5) (end 162.135 102.5) (width 0.25) (layer "B.Cu") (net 15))
 (segment (start 160.835 101.77) (end 160.765 101.7) (width 0.25) (layer "F.Cu") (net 16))
 (segment (start 155.465 101.7) (end 155.165 102) (width 0.25) (layer "F.Cu") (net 16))
 (segment (start 155.165 102) (end 155.01 102) (width 0.25) (layer "F.Cu") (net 16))
 (segment (start 160.765 101.7) (end 155.465 101.7) (width 0.25) (layer "F.Cu") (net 16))
 (via (at 160.765 101.7) (size 0.45) (drill 0.2) (layers "F.Cu" "B.Cu") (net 16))
 (segment (start 160.765 101.7) (end 162.135 101.7) (width 0.25) (layer "B.Cu") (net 16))
 (segment (start 154.535 101.525) (end 154.535 98.27) (width 0.25) (layer "F.Cu") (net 5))
 (segment (start 154.535 98.27) (end 154.825 97.98) (width 0.25) (layer "F.Cu") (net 5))
 (segment (start 152.285 98.6) (end 152.285 97.98) (width 0.25) (layer "F.Cu") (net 4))
 (segment (start 154.035 101.7) (end 154.035 100.35) (width 0.25) (layer "F.Cu") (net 4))
 (segment (start 154.035 100.35) (end 152.285 98.6) (width 0.25) (layer "F.Cu") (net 4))
 (segment (start 153.445 102.69) (end 154.125 102.69) (width 0.254) (layer "F.Cu") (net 1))
 (segment (start 154.125 102.69) (end 154.445 103.01) (width 0.254) (layer "F.Cu") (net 1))
 (segment (start 154.825 103.01) (end 154.835 103) (width 0.254) (layer "F.Cu") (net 1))
 (segment (start 154.445 103.01) (end 154.825 103.01) (width 0.254) (layer "F.Cu") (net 1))
 (segment (start 152.235 103.5) (end 152.635 103.5) (width 0.254) (layer "F.Cu") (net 1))
 (segment (start 156.395 103.33) (end 155.875 103.33) (width 0.25) (layer "F.Cu") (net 1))
 (segment (start 156.165 103.56) (end 156.395 103.33) (width 0.4) (layer "F.Cu") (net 1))
 (segment (start 156.165 104.94) (end 156.165 103.56) (width 0.4) (layer "F.Cu") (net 1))
 (segment (start 144.325 106.32) (end 154.785 106.32) (width 0.4) (layer "F.Cu") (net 1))
 (segment (start 156.165 103.56) (end 156.425 103.3) (width 0.4) (layer "F.Cu") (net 1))
 (segment (start 156.085 105.75) (end 155.885 105.55) (width 0.254) (layer "F.Cu") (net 1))
 (segment (start 155.875 103.33) (end 155.545 103) (width 0.25) (layer "F.Cu") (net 1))
 (segment (start 154.785 106.32) (end 156.165 104.94) (width 0.4) (layer "F.Cu") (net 1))
 (segment (start 155.545 103) (end 154.835 103) (width 0.25) (layer "F.Cu") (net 1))
 (segment (start 156.085 106.42) (end 156.085 105.75) (width 0.254) (layer "F.Cu") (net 1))
 (segment (start 156.425 103.3) (end 160.815 103.3) (width 0.4) (layer "F.Cu") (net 1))
 (segment (start 141.515 102.1) (end 141.515 103.51) (width 0.4) (layer "F.Cu") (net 1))
 (segment (start 141.515 103.51) (end 144.325 106.32) (width 0.4) (layer "F.Cu") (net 1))
 (segment (start 152.635 103.5) (end 153.445 102.69) (width 0.254) (layer "F.Cu") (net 1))
 (via (at 160.815 103.3) (size 0.45) (drill 0.2) (layers "F.Cu" "B.Cu") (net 1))
 (segment (start 160.815 103.3) (end 162.135 103.3) (width 0.25) (layer "B.Cu") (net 1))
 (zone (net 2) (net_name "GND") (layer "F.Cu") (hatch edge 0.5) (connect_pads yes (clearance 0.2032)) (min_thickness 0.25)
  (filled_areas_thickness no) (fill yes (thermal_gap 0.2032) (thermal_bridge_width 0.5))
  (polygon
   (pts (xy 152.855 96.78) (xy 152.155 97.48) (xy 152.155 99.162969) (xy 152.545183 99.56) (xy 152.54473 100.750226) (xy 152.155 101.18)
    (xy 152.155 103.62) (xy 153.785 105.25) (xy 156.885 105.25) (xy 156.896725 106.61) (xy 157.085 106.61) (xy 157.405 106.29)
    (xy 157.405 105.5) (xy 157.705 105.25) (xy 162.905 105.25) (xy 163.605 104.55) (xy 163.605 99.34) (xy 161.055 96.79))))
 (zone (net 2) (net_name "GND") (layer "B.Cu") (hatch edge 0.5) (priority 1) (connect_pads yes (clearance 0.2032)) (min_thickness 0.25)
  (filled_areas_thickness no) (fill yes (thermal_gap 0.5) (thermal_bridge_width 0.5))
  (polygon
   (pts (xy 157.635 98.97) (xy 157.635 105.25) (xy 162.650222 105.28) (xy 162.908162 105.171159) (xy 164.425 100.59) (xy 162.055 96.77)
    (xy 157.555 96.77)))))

